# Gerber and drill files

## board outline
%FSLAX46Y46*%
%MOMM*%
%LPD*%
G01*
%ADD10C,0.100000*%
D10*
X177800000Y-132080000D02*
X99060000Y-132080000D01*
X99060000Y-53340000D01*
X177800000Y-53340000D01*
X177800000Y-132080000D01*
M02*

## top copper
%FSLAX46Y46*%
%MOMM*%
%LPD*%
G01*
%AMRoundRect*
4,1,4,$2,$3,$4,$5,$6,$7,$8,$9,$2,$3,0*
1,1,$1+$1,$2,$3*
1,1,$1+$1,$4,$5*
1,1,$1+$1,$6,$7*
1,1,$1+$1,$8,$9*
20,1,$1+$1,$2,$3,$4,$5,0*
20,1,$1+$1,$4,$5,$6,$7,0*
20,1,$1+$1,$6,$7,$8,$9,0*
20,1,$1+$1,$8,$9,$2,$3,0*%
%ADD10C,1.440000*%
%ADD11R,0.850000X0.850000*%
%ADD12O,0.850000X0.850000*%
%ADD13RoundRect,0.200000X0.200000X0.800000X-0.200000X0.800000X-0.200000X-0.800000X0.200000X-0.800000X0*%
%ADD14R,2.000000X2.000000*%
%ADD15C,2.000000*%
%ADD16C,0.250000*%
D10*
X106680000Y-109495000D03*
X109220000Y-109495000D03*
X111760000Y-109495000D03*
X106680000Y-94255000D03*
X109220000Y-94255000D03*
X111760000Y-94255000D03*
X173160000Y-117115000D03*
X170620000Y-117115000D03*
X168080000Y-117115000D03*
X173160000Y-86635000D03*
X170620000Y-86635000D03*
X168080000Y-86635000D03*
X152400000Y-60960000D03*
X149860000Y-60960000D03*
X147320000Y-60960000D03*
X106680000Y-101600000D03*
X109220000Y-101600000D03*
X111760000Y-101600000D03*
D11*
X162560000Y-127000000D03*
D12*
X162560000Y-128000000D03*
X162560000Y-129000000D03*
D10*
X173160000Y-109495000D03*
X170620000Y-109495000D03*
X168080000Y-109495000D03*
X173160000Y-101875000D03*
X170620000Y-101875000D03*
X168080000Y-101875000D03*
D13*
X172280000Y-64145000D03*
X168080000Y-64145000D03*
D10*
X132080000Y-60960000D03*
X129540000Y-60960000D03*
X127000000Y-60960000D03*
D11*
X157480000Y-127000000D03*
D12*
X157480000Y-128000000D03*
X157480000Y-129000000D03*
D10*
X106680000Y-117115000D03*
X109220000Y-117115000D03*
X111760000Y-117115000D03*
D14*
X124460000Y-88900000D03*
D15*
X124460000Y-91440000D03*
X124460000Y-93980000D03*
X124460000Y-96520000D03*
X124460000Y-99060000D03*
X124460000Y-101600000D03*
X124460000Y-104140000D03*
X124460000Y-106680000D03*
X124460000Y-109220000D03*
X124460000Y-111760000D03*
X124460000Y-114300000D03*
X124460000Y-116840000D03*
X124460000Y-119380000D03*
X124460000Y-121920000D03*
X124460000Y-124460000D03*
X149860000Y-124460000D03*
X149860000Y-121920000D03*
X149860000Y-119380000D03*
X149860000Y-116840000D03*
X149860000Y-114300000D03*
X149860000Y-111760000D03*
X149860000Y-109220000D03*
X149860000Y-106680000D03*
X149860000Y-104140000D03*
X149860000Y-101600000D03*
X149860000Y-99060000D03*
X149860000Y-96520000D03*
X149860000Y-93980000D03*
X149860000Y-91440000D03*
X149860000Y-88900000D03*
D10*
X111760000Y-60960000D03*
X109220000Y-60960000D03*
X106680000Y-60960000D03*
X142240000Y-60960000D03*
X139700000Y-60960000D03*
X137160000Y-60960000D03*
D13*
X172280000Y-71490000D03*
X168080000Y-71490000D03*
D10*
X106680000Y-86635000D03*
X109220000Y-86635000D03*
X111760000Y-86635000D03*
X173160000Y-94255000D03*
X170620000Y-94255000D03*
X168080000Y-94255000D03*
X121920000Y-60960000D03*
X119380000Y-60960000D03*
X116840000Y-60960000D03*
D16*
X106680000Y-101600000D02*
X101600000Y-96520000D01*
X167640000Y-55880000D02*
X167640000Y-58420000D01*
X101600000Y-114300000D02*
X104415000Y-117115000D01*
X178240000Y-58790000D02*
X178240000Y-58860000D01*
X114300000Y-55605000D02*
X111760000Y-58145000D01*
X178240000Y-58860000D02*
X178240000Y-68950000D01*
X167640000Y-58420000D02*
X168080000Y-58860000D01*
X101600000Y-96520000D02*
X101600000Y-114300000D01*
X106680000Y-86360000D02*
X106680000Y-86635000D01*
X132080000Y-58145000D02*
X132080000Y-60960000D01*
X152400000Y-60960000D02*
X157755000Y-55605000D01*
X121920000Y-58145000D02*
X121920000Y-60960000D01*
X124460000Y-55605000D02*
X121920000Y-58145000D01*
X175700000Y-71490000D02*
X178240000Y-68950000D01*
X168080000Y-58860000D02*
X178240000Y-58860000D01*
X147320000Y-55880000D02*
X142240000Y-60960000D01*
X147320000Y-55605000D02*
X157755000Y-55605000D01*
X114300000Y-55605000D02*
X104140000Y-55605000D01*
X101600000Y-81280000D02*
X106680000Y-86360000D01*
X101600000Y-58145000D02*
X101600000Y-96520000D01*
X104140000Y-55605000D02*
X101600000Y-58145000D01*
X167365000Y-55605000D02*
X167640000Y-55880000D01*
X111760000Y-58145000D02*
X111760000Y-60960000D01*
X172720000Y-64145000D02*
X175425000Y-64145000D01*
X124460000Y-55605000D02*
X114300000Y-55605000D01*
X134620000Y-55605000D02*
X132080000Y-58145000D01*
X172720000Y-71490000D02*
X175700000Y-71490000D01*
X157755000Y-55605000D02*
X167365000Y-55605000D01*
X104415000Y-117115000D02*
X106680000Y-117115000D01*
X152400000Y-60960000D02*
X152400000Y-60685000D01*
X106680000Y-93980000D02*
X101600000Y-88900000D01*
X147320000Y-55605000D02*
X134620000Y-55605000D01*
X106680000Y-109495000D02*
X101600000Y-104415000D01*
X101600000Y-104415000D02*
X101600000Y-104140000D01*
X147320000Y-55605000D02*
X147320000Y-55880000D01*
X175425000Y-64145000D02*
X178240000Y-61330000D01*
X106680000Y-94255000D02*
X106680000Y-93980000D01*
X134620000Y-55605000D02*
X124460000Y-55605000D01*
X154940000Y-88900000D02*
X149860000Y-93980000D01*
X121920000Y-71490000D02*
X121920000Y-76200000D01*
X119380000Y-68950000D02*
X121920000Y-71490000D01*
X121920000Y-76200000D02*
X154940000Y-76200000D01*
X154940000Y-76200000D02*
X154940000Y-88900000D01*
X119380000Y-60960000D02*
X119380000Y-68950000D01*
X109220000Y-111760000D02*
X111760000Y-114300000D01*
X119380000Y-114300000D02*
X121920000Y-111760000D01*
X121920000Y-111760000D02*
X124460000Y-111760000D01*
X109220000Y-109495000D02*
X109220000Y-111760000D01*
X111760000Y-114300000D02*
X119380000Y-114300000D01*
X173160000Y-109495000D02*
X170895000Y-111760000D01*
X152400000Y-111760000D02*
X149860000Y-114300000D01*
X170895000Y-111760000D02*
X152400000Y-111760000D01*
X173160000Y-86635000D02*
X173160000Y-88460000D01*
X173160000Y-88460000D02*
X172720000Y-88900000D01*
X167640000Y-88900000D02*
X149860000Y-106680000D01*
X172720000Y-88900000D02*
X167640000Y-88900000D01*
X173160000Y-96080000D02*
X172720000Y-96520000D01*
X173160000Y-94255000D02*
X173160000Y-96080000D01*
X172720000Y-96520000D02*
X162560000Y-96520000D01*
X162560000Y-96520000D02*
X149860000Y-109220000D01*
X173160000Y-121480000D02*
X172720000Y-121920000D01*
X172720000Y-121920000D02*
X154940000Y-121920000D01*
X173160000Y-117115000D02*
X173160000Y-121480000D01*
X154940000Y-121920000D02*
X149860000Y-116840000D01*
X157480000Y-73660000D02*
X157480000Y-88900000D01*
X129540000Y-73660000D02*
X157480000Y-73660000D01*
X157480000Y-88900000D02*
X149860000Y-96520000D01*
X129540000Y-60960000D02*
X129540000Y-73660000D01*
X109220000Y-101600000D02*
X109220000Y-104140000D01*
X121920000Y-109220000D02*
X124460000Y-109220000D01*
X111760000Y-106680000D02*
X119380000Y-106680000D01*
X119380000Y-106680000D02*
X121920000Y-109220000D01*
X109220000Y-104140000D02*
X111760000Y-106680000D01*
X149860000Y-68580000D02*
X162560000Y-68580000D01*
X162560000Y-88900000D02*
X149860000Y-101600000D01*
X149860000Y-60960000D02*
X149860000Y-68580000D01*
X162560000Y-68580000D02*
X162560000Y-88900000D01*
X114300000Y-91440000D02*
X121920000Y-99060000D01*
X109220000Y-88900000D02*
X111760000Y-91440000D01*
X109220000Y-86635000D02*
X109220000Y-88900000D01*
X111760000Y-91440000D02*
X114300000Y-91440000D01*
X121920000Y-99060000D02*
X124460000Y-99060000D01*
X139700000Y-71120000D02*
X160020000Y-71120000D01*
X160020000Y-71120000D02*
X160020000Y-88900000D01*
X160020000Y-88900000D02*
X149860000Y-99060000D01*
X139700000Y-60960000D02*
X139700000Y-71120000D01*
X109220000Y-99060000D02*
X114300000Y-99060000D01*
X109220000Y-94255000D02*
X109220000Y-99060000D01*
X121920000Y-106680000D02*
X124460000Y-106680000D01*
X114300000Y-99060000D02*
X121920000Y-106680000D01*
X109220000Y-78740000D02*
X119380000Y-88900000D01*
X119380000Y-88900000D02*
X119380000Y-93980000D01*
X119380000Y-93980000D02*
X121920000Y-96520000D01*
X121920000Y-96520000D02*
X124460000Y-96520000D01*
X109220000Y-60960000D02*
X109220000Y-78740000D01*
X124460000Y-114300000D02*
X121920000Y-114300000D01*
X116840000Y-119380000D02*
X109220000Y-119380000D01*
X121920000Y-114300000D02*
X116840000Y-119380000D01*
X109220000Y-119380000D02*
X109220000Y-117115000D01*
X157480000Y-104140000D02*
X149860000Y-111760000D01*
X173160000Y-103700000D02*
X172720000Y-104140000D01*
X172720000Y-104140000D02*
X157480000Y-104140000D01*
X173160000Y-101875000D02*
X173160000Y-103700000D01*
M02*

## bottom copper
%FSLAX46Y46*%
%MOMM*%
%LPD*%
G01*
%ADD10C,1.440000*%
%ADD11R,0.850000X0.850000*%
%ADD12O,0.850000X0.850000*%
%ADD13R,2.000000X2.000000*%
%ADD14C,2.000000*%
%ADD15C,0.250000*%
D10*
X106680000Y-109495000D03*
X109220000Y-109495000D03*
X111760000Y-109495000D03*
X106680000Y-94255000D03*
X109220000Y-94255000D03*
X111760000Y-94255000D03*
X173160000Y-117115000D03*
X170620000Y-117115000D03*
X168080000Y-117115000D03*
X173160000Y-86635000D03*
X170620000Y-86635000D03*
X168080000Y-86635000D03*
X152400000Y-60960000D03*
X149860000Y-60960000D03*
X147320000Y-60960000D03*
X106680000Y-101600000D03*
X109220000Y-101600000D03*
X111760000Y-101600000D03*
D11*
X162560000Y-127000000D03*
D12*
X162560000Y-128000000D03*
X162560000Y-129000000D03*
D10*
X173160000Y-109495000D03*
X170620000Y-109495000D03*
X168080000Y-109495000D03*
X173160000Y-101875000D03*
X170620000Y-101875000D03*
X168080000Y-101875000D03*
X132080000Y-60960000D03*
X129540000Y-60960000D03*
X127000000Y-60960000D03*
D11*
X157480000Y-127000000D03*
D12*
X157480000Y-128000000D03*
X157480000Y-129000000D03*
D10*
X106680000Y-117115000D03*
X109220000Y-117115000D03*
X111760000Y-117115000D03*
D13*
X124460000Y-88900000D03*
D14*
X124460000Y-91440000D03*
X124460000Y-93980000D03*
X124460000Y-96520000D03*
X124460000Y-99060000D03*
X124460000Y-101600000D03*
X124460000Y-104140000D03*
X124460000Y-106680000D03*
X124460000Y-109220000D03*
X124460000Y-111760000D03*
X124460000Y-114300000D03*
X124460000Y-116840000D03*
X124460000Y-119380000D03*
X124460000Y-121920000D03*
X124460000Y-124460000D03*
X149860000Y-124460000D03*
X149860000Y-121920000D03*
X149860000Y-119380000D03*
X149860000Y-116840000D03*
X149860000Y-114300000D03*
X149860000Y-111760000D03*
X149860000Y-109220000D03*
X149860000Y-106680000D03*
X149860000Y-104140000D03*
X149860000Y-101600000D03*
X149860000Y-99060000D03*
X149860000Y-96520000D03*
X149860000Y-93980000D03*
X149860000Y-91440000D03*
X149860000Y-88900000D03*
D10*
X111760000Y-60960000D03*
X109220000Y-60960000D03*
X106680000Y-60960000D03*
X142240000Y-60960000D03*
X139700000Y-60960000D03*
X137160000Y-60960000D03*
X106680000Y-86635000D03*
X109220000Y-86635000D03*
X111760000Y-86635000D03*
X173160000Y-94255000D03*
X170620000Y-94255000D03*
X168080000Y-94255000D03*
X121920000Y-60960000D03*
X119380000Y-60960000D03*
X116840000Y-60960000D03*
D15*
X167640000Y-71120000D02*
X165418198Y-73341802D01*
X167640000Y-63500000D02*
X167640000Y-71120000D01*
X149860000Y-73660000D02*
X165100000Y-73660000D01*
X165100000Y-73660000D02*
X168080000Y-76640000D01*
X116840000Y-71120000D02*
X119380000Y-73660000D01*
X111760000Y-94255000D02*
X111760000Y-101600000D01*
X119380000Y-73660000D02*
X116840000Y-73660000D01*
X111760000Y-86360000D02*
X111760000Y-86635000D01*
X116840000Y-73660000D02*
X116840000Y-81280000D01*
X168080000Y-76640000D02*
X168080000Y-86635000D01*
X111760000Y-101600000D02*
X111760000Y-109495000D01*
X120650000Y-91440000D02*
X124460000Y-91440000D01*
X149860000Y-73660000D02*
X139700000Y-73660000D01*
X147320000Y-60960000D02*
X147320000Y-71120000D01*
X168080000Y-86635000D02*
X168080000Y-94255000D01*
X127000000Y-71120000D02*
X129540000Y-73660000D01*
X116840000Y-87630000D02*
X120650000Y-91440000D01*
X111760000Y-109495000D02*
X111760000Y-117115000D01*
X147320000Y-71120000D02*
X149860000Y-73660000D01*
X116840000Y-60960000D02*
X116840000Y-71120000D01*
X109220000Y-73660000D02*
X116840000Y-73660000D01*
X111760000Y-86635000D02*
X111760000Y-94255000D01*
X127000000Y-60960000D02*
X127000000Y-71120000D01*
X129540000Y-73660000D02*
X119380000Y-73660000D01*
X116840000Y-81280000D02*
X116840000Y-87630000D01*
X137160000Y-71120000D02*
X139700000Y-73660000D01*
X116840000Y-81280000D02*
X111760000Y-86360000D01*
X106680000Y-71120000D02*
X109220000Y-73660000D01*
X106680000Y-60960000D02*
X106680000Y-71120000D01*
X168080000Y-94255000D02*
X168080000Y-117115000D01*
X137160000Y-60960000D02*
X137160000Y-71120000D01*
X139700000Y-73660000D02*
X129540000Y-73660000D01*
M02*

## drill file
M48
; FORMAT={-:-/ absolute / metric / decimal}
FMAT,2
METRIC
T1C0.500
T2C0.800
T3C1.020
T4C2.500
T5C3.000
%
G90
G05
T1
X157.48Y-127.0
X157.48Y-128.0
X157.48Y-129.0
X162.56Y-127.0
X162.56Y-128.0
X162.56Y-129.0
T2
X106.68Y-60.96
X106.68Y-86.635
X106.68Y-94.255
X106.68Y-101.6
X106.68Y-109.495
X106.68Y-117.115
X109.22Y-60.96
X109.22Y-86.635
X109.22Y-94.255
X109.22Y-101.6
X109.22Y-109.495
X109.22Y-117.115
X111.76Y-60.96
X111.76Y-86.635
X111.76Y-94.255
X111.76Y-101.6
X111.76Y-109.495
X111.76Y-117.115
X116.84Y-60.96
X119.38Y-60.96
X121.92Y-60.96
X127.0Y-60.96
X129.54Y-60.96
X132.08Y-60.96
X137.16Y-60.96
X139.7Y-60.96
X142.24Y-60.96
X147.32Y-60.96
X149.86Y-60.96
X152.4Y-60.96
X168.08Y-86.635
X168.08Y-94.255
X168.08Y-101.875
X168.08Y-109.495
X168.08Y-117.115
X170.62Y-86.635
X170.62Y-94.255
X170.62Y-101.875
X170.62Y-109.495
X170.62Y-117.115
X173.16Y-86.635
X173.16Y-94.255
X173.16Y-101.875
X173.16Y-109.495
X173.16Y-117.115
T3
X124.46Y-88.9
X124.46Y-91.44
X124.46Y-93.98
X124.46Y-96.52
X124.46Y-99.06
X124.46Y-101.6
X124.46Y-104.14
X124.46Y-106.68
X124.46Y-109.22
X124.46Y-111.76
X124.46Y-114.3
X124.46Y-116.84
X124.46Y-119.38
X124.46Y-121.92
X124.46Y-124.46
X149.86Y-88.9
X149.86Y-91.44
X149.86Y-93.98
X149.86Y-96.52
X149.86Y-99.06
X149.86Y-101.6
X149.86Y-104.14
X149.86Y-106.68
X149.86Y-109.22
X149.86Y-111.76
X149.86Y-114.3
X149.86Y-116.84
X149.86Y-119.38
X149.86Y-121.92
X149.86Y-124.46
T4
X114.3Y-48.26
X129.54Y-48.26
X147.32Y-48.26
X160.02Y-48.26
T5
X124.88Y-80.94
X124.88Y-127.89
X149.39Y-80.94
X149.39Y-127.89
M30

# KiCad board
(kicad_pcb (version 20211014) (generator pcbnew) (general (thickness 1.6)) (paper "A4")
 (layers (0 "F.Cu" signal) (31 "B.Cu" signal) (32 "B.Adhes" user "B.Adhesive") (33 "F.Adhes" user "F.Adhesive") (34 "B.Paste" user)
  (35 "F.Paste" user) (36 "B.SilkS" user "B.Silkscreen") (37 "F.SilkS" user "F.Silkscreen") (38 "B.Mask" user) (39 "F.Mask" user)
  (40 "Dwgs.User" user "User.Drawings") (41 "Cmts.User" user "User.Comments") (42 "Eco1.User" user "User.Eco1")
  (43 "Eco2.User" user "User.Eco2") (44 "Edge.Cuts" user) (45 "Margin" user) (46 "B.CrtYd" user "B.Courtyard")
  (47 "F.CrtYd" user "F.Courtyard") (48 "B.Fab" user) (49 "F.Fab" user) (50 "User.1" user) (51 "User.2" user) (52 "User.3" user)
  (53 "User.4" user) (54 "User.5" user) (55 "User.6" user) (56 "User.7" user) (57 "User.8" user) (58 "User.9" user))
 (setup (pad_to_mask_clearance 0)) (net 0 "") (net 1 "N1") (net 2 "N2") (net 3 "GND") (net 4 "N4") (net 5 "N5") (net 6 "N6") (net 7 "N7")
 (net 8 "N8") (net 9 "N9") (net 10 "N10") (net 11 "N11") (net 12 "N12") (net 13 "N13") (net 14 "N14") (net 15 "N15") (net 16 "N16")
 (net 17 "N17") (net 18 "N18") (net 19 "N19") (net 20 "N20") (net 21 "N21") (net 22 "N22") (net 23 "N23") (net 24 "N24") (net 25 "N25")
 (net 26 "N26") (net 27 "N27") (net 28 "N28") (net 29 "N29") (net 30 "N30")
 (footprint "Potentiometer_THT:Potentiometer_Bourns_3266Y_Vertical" (layer "F.Cu") (at 106.68 109.495 180)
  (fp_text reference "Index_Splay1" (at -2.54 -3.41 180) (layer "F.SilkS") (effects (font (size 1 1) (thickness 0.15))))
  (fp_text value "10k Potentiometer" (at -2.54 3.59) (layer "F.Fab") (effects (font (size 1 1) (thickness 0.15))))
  (pad "1" thru_hole circle (at 0 0 180) (size 1.44 1.44) (drill 0.8) (layers *.Cu *.Mask) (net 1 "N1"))
  (pad "2" thru_hole circle (at -2.54 0 180) (size 1.44 1.44) (drill 0.8) (layers *.Cu *.Mask) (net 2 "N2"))
  (pad "3" thru_hole circle (at -5.08 0 180) (size 1.44 1.44) (drill 0.8) (layers *.Cu *.Mask) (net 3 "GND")))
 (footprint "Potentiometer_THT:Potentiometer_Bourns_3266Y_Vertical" (layer "F.Cu") (at 106.68 94.255 180)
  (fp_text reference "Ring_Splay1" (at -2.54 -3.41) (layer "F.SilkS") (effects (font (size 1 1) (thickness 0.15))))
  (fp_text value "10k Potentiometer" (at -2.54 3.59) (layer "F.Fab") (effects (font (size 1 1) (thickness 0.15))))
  (pad "1" thru_hole circle (at 0 0 180) (size 1.44 1.44) (drill 0.8) (layers *.Cu *.Mask) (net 1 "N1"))
  (pad "2" thru_hole circle (at -2.54 0 180) (size 1.44 1.44) (drill 0.8) (layers *.Cu *.Mask) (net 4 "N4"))
  (pad "3" thru_hole circle (at -5.08 0 180) (size 1.44 1.44) (drill 0.8) (layers *.Cu *.Mask) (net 3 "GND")))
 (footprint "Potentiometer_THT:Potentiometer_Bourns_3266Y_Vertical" (layer "F.Cu") (at 173.16 117.115)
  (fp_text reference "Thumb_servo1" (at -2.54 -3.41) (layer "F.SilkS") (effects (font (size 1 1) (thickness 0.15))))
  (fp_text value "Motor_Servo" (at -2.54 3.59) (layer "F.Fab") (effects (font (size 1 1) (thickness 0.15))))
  (pad "1" thru_hole circle (at 0 0) (size 1.44 1.44) (drill 0.8) (layers *.Cu *.Mask) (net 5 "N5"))
  (pad "2" thru_hole circle (at -2.54 0) (size 1.44 1.44) (drill 0.8) (layers *.Cu *.Mask) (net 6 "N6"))
  (pad "3" thru_hole circle (at -5.08 0) (size 1.44 1.44) (drill 0.8) (layers *.Cu *.Mask) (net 3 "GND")))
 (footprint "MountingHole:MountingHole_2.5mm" (layer "F.Cu") (at 160.02 48.26)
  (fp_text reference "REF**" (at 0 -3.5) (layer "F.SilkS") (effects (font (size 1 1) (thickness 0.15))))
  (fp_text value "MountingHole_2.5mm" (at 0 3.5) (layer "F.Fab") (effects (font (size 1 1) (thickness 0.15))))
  (pad "" np_thru_hole circle (at 0 0) (size 2.5 2.5) (drill 2.5) (layers *.Cu *.Mask)))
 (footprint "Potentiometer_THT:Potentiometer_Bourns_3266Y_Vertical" (layer "F.Cu") (at 173.16 86.635)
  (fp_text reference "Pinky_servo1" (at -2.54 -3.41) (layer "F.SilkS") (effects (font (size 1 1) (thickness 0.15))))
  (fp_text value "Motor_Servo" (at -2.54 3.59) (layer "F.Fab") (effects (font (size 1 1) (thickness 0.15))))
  (pad "1" thru_hole circle (at 0 0) (size 1.44 1.44) (drill 0.8) (layers *.Cu *.Mask) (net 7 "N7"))
  (pad "2" thru_hole circle (at -2.54 0) (size 1.44 1.44) (drill 0.8) (layers *.Cu *.Mask) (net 6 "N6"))
  (pad "3" thru_hole circle (at -5.08 0) (size 1.44 1.44) (drill 0.8) (layers *.Cu *.Mask) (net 3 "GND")))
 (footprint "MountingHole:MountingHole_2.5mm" (layer "F.Cu") (at 114.3 48.26)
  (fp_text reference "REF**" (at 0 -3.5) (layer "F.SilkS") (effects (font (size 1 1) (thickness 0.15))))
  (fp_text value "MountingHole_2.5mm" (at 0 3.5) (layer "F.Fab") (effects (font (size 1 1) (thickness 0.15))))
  (pad "" np_thru_hole circle (at 0 0) (size 2.5 2.5) (drill 2.5) (layers *.Cu *.Mask)))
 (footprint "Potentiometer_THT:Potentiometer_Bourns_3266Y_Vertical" (layer "F.Cu") (at 152.4 60.96)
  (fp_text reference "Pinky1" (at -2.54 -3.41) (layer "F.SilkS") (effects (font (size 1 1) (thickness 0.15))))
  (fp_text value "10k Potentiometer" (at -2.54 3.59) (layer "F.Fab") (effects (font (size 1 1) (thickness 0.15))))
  (pad "1" thru_hole circle (at 0 0) (size 1.44 1.44) (drill 0.8) (layers *.Cu *.Mask) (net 1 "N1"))
  (pad "2" thru_hole circle (at -2.54 0) (size 1.44 1.44) (drill 0.8) (layers *.Cu *.Mask) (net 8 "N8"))
  (pad "3" thru_hole circle (at -5.08 0) (size 1.44 1.44) (drill 0.8) (layers *.Cu *.Mask) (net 3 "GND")))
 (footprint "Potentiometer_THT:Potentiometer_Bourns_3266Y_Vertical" (layer "F.Cu") (at 106.68 101.6 180)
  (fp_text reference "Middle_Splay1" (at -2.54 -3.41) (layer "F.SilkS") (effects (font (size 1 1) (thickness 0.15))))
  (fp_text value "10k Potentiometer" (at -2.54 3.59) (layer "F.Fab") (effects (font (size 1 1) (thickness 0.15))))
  (pad "1" thru_hole circle (at 0 0 180) (size 1.44 1.44) (drill 0.8) (layers *.Cu *.Mask) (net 1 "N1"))
  (pad "2" thru_hole circle (at -2.54 0 180) (size 1.44 1.44) (drill 0.8) (layers *.Cu *.Mask) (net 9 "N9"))
  (pad "3" thru_hole circle (at -5.08 0 180) (size 1.44 1.44) (drill 0.8) (layers *.Cu *.Mask) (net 3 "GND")))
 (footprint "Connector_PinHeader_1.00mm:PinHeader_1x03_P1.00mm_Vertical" (layer "F.Cu") (at 162.56 127)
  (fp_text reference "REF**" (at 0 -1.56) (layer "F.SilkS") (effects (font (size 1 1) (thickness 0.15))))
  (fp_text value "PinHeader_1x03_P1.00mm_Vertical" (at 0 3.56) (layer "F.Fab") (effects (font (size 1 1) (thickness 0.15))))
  (pad "1" thru_hole rect (at 0 0) (size 0.85 0.85) (drill 0.5) (layers *.Cu *.Mask))
  (pad "2" thru_hole oval (at 0 1) (size 0.85 0.85) (drill 0.5) (layers *.Cu *.Mask))
  (pad "3" thru_hole oval (at 0 2) (size 0.85 0.85) (drill 0.5) (layers *.Cu *.Mask)))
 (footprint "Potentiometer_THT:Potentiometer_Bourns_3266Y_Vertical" (layer "F.Cu") (at 173.16 109.495)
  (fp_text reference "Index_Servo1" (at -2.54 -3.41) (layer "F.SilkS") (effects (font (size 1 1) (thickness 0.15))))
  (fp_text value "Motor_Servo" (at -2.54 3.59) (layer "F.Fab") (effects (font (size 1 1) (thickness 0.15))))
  (pad "1" thru_hole circle (at 0 0) (size 1.44 1.44) (drill 0.8) (layers *.Cu *.Mask) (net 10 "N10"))
  (pad "2" thru_hole circle (at -2.54 0) (size 1.44 1.44) (drill 0.8) (layers *.Cu *.Mask) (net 6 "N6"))
  (pad "3" thru_hole circle (at -5.08 0) (size 1.44 1.44) (drill 0.8) (layers *.Cu *.Mask) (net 3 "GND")))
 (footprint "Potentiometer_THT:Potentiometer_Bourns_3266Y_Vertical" (layer "F.Cu") (at 173.16 101.875)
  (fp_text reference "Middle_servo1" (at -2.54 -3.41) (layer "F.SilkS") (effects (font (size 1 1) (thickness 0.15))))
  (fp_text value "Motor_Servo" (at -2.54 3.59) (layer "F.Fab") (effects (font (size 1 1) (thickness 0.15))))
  (pad "1" thru_hole circle (at 0 0) (size 1.44 1.44) (drill 0.8) (layers *.Cu *.Mask) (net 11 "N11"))
  (pad "2" thru_hole circle (at -2.54 0) (size 1.44 1.44) (drill 0.8) (layers *.Cu *.Mask) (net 6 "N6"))
  (pad "3" thru_hole circle (at -5.08 0) (size 1.44 1.44) (drill 0.8) (layers *.Cu *.Mask) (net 3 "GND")))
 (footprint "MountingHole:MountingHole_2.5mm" (layer "F.Cu") (at 147.32 48.26)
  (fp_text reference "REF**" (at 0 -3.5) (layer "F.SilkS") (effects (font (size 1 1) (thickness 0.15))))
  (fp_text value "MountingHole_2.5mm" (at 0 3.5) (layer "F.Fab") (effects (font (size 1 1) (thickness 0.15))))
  (pad "" np_thru_hole circle (at 0 0) (size 2.5 2.5) (drill 2.5) (layers *.Cu *.Mask)))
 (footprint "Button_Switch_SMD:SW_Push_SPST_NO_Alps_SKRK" (layer "F.Cu") (at 170.18 64.145 180)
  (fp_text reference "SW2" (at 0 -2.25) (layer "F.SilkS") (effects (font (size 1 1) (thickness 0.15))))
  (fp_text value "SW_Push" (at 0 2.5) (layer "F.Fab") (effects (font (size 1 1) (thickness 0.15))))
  (pad "1" smd roundrect (at -2.1 0 180) (size 0.8 2) (layers "F.Cu" "F.Paste" "F.Mask") (roundrect_rratio 0.25) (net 1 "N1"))
  (pad "2" smd roundrect (at 2.1 0 180) (size 0.8 2) (layers "F.Cu" "F.Paste" "F.Mask") (roundrect_rratio 0.25) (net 3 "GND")))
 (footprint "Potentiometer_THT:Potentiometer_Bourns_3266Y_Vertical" (layer "F.Cu") (at 132.08 60.96)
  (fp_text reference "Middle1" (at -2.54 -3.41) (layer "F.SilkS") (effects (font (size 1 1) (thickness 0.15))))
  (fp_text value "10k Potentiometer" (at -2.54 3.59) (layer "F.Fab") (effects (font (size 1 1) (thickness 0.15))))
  (pad "1" thru_hole circle (at 0 0) (size 1.44 1.44) (drill 0.8) (layers *.Cu *.Mask) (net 1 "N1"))
  (pad "2" thru_hole circle (at -2.54 0) (size 1.44 1.44) (drill 0.8) (layers *.Cu *.Mask) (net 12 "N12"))
  (pad "3" thru_hole circle (at -5.08 0) (size 1.44 1.44) (drill 0.8) (layers *.Cu *.Mask) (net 3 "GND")))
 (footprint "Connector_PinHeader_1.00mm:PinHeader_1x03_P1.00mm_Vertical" (layer "F.Cu") (at 157.48 127)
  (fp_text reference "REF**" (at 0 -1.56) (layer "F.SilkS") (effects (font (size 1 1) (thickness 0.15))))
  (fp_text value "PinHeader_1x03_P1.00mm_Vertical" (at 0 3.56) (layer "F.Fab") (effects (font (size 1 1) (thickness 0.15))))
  (pad "1" thru_hole rect (at 0 0) (size 0.85 0.85) (drill 0.5) (layers *.Cu *.Mask))
  (pad "2" thru_hole oval (at 0 1) (size 0.85 0.85) (drill 0.5) (layers *.Cu *.Mask))
  (pad "3" thru_hole oval (at 0 2) (size 0.85 0.85) (drill 0.5) (layers *.Cu *.Mask)))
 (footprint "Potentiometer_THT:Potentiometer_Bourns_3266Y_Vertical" (layer "F.Cu") (at 106.68 117.115 180)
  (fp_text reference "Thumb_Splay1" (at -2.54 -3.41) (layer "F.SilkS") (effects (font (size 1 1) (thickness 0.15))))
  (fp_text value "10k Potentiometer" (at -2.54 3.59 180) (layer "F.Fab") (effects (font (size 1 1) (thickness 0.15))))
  (pad "1" thru_hole circle (at 0 0 180) (size 1.44 1.44) (drill 0.8) (layers *.Cu *.Mask) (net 1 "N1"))
  (pad "2" thru_hole circle (at -2.54 0 180) (size 1.44 1.44) (drill 0.8) (layers *.Cu *.Mask) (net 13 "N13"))
  (pad "3" thru_hole circle (at -5.08 0 180) (size 1.44 1.44) (drill 0.8) (layers *.Cu *.Mask) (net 3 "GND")))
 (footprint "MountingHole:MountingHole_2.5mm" (layer "F.Cu") (at 129.54 48.26)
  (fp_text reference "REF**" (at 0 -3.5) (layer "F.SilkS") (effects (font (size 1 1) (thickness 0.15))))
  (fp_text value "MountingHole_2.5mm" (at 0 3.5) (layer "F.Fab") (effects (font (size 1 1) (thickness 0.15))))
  (pad "" np_thru_hole circle (at 0 0) (size 2.5 2.5) (drill 2.5) (layers *.Cu *.Mask)))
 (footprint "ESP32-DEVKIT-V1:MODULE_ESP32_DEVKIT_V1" (layer "F.Cu") (at 137.16 104.415)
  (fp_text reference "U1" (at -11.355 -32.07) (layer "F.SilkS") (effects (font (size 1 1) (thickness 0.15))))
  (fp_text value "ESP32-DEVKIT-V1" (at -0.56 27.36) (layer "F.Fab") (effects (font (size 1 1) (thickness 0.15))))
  (pad "" np_thru_hole circle (at -12.28 -23.475) (size 3 3) (drill 3) (layers *.Cu *.Mask))
  (pad "" np_thru_hole circle (at 12.23 23.475) (size 3 3) (drill 3) (layers *.Cu *.Mask))
  (pad "" np_thru_hole circle (at 12.23 -23.475) (size 3 3) (drill 3) (layers *.Cu *.Mask))
  (pad "" np_thru_hole circle (at -12.28 23.475) (size 3 3) (drill 3) (layers *.Cu *.Mask))
  (pad "1" thru_hole rect (at -12.7 -15.515) (size 2 2) (drill 1.02) (layers *.Cu *.Mask) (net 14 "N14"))
  (pad "2" thru_hole circle (at -12.7 -12.975) (size 2 2) (drill 1.02) (layers *.Cu *.Mask) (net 3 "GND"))
  (pad "3" thru_hole circle (at -12.7 -10.435) (size 2 2) (drill 1.02) (layers *.Cu *.Mask) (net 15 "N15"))
  (pad "4" thru_hole circle (at -12.7 -7.895) (size 2 2) (drill 1.02) (layers *.Cu *.Mask) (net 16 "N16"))
  (pad "5" thru_hole circle (at -12.7 -5.355) (size 2 2) (drill 1.02) (layers *.Cu *.Mask) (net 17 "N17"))
  (pad "6" thru_hole circle (at -12.7 -2.815) (size 2 2) (drill 1.02) (layers *.Cu *.Mask) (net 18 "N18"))
  (pad "7" thru_hole circle (at -12.7 -0.275) (size 2 2) (drill 1.02) (layers *.Cu *.Mask) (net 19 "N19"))
  (pad "8" thru_hole circle (at -12.7 2.265) (size 2 2) (drill 1.02) (layers *.Cu *.Mask) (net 4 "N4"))
  (pad "9" thru_hole circle (at -12.7 4.805) (size 2 2) (drill 1.02) (layers *.Cu *.Mask) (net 9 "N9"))
  (pad "10" thru_hole circle (at -12.7 7.345) (size 2 2) (drill 1.02) (layers *.Cu *.Mask) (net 2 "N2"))
  (pad "11" thru_hole circle (at -12.7 9.885) (size 2 2) (drill 1.02) (layers *.Cu *.Mask) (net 13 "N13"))
  (pad "12" thru_hole circle (at -12.7 12.425) (size 2 2) (drill 1.02) (layers *.Cu *.Mask) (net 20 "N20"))
  (pad "13" thru_hole circle (at -12.7 14.965) (size 2 2) (drill 1.02) (layers *.Cu *.Mask) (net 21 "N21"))
  (pad "14" thru_hole circle (at -12.7 17.505) (size 2 2) (drill 1.02) (layers *.Cu *.Mask) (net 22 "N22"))
  (pad "15" thru_hole circle (at -12.7 20.045) (size 2 2) (drill 1.02) (layers *.Cu *.Mask) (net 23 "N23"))
  (pad "16" thru_hole circle (at 12.7 20.045) (size 2 2) (drill 1.02) (layers *.Cu *.Mask) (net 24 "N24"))
  (pad "17" thru_hole circle (at 12.7 17.505) (size 2 2) (drill 1.02) (layers *.Cu *.Mask) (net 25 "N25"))
  (pad "18" thru_hole circle (at 12.7 14.965) (size 2 2) (drill 1.02) (layers *.Cu *.Mask) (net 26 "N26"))
  (pad "19" thru_hole circle (at 12.7 12.425) (size 2 2) (drill 1.02) (layers *.Cu *.Mask) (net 5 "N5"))
  (pad "20" thru_hole circle (at 12.7 9.885) (size 2 2) (drill 1.02) (layers *.Cu *.Mask) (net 10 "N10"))
  (pad "21" thru_hole circle (at 12.7 7.345) (size 2 2) (drill 1.02) (layers *.Cu *.Mask) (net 11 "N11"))
  (pad "22" thru_hole circle (at 12.7 4.805) (size 2 2) (drill 1.02) (layers *.Cu *.Mask) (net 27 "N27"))
  (pad "23" thru_hole circle (at 12.7 2.265) (size 2 2) (drill 1.02) (layers *.Cu *.Mask) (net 7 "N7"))
  (pad "24" thru_hole circle (at 12.7 -0.275) (size 2 2) (drill 1.02) (layers *.Cu *.Mask) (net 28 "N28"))
  (pad "25" thru_hole circle (at 12.7 -2.815) (size 2 2) (drill 1.02) (layers *.Cu *.Mask) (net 8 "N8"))
  (pad "26" thru_hole circle (at 12.7 -5.355) (size 2 2) (drill 1.02) (layers *.Cu *.Mask) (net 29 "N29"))
  (pad "27" thru_hole circle (at 12.7 -7.895) (size 2 2) (drill 1.02) (layers *.Cu *.Mask) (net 12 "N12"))
  (pad "28" thru_hole circle (at 12.7 -10.435) (size 2 2) (drill 1.02) (layers *.Cu *.Mask) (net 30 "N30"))
  (pad "29" thru_hole circle (at 12.7 -12.975) (size 2 2) (drill 1.02) (layers *.Cu *.Mask) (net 3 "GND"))
  (pad "30" thru_hole circle (at 12.7 -15.515) (size 2 2) (drill 1.02) (layers *.Cu *.Mask) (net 1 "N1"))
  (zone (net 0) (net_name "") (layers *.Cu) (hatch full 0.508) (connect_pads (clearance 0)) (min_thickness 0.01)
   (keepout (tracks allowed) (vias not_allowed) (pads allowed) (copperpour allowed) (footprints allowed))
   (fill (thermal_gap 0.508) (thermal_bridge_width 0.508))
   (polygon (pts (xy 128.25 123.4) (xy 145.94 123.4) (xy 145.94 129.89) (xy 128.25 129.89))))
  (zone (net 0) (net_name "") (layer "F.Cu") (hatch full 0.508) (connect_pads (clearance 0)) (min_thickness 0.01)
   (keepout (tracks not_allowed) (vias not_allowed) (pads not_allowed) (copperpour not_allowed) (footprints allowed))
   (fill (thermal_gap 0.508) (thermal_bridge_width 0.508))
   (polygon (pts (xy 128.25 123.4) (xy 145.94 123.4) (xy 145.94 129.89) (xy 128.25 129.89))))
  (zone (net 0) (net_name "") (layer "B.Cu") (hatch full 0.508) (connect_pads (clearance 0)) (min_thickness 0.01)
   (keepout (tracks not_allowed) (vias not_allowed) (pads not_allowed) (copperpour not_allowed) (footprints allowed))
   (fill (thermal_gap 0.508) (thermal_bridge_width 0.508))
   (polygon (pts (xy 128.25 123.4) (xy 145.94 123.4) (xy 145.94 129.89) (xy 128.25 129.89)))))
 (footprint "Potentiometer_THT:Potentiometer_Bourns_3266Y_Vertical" (layer "F.Cu") (at 111.76 60.96)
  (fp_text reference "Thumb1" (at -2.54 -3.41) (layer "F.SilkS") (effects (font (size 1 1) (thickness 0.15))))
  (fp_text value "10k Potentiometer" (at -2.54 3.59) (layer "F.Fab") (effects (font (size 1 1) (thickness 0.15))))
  (pad "1" thru_hole circle (at 0 0) (size 1.44 1.44) (drill 0.8) (layers *.Cu *.Mask) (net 1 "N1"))
  (pad "2" thru_hole circle (at -2.54 0) (size 1.44 1.44) (drill 0.8) (layers *.Cu *.Mask) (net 16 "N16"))
  (pad "3" thru_hole circle (at -5.08 0) (size 1.44 1.44) (drill 0.8) (layers *.Cu *.Mask) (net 3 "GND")))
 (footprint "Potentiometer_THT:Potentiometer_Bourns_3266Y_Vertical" (layer "F.Cu") (at 142.24 60.96)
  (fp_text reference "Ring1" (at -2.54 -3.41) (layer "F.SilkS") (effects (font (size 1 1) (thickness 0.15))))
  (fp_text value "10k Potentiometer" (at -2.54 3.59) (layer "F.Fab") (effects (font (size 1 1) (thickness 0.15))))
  (pad "1" thru_hole circle (at 0 0) (size 1.44 1.44) (drill 0.8) (layers *.Cu *.Mask) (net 1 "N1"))
  (pad "2" thru_hole circle (at -2.54 0) (size 1.44 1.44) (drill 0.8) (layers *.Cu *.Mask) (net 29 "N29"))
  (pad "3" thru_hole circle (at -5.08 0) (size 1.44 1.44) (drill 0.8) (layers *.Cu *.Mask) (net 3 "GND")))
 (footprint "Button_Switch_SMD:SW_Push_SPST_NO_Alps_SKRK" (layer "F.Cu") (at 170.18 71.49 180)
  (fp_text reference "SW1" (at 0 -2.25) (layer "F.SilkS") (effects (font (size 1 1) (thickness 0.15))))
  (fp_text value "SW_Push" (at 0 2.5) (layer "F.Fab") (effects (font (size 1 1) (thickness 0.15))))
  (pad "1" smd roundrect (at -2.1 0 180) (size 0.8 2) (layers "F.Cu" "F.Paste" "F.Mask") (roundrect_rratio 0.25) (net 1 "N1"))
  (pad "2" smd roundrect (at 2.1 0 180) (size 0.8 2) (layers "F.Cu" "F.Paste" "F.Mask") (roundrect_rratio 0.25) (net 3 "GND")))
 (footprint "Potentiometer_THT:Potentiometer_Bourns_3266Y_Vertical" (layer "F.Cu") (at 106.68 86.635 180)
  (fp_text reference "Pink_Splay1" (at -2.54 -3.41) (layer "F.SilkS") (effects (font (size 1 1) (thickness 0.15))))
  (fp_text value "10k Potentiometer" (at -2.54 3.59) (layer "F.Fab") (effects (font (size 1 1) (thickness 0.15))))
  (pad "1" thru_hole circle (at 0 0 180) (size 1.44 1.44) (drill 0.8) (layers *.Cu *.Mask) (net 1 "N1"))
  (pad "2" thru_hole circle (at -2.54 0 180) (size 1.44 1.44) (drill 0.8) (layers *.Cu *.Mask) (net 17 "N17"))
  (pad "3" thru_hole circle (at -5.08 0 180) (size 1.44 1.44) (drill 0.8) (layers *.Cu *.Mask) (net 3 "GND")))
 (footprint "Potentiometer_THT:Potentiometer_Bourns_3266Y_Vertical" (layer "F.Cu") (at 173.16 94.255)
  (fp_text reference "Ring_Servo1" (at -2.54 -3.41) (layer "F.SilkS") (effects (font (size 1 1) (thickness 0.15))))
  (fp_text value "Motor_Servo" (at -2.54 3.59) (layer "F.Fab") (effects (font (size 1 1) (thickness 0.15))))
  (pad "1" thru_hole circle (at 0 0) (size 1.44 1.44) (drill 0.8) (layers *.Cu *.Mask) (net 27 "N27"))
  (pad "2" thru_hole circle (at -2.54 0) (size 1.44 1.44) (drill 0.8) (layers *.Cu *.Mask) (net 6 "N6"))
  (pad "3" thru_hole circle (at -5.08 0) (size 1.44 1.44) (drill 0.8) (layers *.Cu *.Mask) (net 3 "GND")))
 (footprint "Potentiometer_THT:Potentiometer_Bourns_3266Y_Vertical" (layer "F.Cu") (at 121.92 60.96)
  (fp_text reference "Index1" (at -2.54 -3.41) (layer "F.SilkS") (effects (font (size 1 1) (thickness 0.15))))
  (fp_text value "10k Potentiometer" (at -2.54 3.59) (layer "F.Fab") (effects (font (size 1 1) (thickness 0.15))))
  (pad "1" thru_hole circle (at 0 0) (size 1.44 1.44) (drill 0.8) (layers *.Cu *.Mask) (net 1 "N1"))
  (pad "2" thru_hole circle (at -2.54 0) (size 1.44 1.44) (drill 0.8) (layers *.Cu *.Mask) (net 30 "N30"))
  (pad "3" thru_hole circle (at -5.08 0) (size 1.44 1.44) (drill 0.8) (layers *.Cu *.Mask) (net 3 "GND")))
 (gr_poly (pts (xy 177.8 132.08) (xy 99.06 132.08) (xy 99.06 53.34) (xy 177.8 53.34)) (layer "Edge.Cuts") (width 0.1) (fill none))
 (segment (start 167.64 71.12) (end 165.418198 73.341802) (width 0.25) (layer "B.Cu") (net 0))
 (segment (start 167.64 63.5) (end 167.64 71.12) (width 0.25) (layer "B.Cu") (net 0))
 (segment (start 106.68 101.6) (end 101.6 96.52) (width 0.25) (layer "F.Cu") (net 1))
 (segment (start 167.64 55.88) (end 167.64 58.42) (width 0.25) (layer "F.Cu") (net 1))
 (segment (start 101.6 114.3) (end 104.415 117.115) (width 0.25) (layer "F.Cu") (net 1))
 (segment (start 178.24 58.79) (end 178.24 58.86) (width 0.25) (layer "F.Cu") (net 1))
 (segment (start 114.3 55.605) (end 111.76 58.145) (width 0.25) (layer "F.Cu") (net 1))
 (segment (start 178.24 58.86) (end 178.24 68.95) (width 0.25) (layer "F.Cu") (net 1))
 (segment (start 167.64 58.42) (end 168.08 58.86) (width 0.25) (layer "F.Cu") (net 1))
 (segment (start 101.6 96.52) (end 101.6 114.3) (width 0.25) (layer "F.Cu") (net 1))
 (segment (start 106.68 86.36) (end 106.68 86.635) (width 0.25) (layer "F.Cu") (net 1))
 (segment (start 132.08 58.145) (end 132.08 60.96) (width 0.25) (layer "F.Cu") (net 1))
 (segment (start 152.4 60.96) (end 157.755 55.605) (width 0.25) (layer "F.Cu") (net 1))
 (segment (start 121.92 58.145) (end 121.92 60.96) (width 0.25) (layer "F.Cu") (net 1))
 (segment (start 124.46 55.605) (end 121.92 58.145) (width 0.25) (layer "F.Cu") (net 1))
 (segment (start 175.7 71.49) (end 178.24 68.95) (width 0.25) (layer "F.Cu") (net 1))
 (segment (start 168.08 58.86) (end 178.24 58.86) (width 0.25) (layer "F.Cu") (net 1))
 (segment (start 147.32 55.88) (end 142.24 60.96) (width 0.25) (layer "F.Cu") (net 1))
 (segment (start 147.32 55.605) (end 157.755 55.605) (width 0.25) (layer "F.Cu") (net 1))
 (segment (start 114.3 55.605) (end 104.14 55.605) (width 0.25) (layer "F.Cu") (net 1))
 (segment (start 101.6 81.28) (end 106.68 86.36) (width 0.25) (layer "F.Cu") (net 1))
 (segment (start 101.6 58.145) (end 101.6 96.52) (width 0.25) (layer "F.Cu") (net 1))
 (segment (start 104.14 55.605) (end 101.6 58.145) (width 0.25) (layer "F.Cu") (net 1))
 (segment (start 167.365 55.605) (end 167.64 55.88) (width 0.25) (layer "F.Cu") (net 1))
 (segment (start 111.76 58.145) (end 111.76 60.96) (width 0.25) (layer "F.Cu") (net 1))
 (segment (start 172.72 64.145) (end 175.425 64.145) (width 0.25) (layer "F.Cu") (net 1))
 (segment (start 124.46 55.605) (end 114.3 55.605) (width 0.25) (layer "F.Cu") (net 1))
 (segment (start 134.62 55.605) (end 132.08 58.145) (width 0.25) (layer "F.Cu") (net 1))
 (segment (start 172.72 71.49) (end 175.7 71.49) (width 0.25) (layer "F.Cu") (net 1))
 (segment (start 157.755 55.605) (end 167.365 55.605) (width 0.25) (layer "F.Cu") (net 1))
 (segment (start 104.415 117.115) (end 106.68 117.115) (width 0.25) (layer "F.Cu") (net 1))
 (segment (start 152.4 60.96) (end 152.4 60.685) (width 0.25) (layer "F.Cu") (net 1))
 (segment (start 106.68 93.98) (end 101.6 88.9) (width 0.25) (layer "F.Cu") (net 1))
 (segment (start 147.32 55.605) (end 134.62 55.605) (width 0.25) (layer "F.Cu") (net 1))
 (segment (start 106.68 109.495) (end 101.6 104.415) (width 0.25) (layer "F.Cu") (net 1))
 (segment (start 101.6 104.415) (end 101.6 104.14) (width 0.25) (layer "F.Cu") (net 1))
 (segment (start 147.32 55.605) (end 147.32 55.88) (width 0.25) (layer "F.Cu") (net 1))
 (segment (start 175.425 64.145) (end 178.24 61.33) (width 0.25) (layer "F.Cu") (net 1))
 (segment (start 106.68 94.255) (end 106.68 93.98) (width 0.25) (layer "F.Cu") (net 1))
 (segment (start 134.62 55.605) (end 124.46 55.605) (width 0.25) (layer "F.Cu") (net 1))
 (segment (start 154.94 88.9) (end 149.86 93.98) (width 0.25) (layer "F.Cu") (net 30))
 (segment (start 121.92 71.49) (end 121.92 76.2) (width 0.25) (layer "F.Cu") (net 30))
 (segment (start 119.38 68.95) (end 121.92 71.49) (width 0.25) (layer "F.Cu") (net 30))
 (segment (start 121.92 76.2) (end 154.94 76.2) (width 0.25) (layer "F.Cu") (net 30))
 (segment (start 154.94 76.2) (end 154.94 88.9) (width 0.25) (layer "F.Cu") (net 30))
 (segment (start 119.38 60.96) (end 119.38 68.95) (width 0.25) (layer "F.Cu") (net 30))
 (segment (start 149.86 73.66) (end 165.1 73.66) (width 0.25) (layer "B.Cu") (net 3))
 (segment (start 165.1 73.66) (end 168.08 76.64) (width 0.25) (layer "B.Cu") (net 3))
 (segment (start 116.84 71.12) (end 119.38 73.66) (width 0.25) (layer "B.Cu") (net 3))
 (segment (start 111.76 94.255) (end 111.76 101.6) (width 0.25) (layer "B.Cu") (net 3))
 (segment (start 119.38 73.66) (end 116.84 73.66) (width 0.25) (layer "B.Cu") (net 3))
 (segment (start 111.76 86.36) (end 111.76 86.635) (width 0.25) (layer "B.Cu") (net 3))
 (segment (start 116.84 73.66) (end 116.84 81.28) (width 0.25) (layer "B.Cu") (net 3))
 (segment (start 168.08 76.64) (end 168.08 86.635) (width 0.25) (layer "B.Cu") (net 3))
 (segment (start 111.76 101.6) (end 111.76 109.495) (width 0.25) (layer "B.Cu") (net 3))
 (segment (start 120.65 91.44) (end 124.46 91.44) (width 0.25) (layer "B.Cu") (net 3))
 (segment (start 149.86 73.66) (end 139.7 73.66) (width 0.25) (layer "B.Cu") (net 3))
 (segment (start 147.32 60.96) (end 147.32 71.12) (width 0.25) (layer "B.Cu") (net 3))
 (segment (start 168.08 86.635) (end 168.08 94.255) (width 0.25) (layer "B.Cu") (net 3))
 (segment (start 127 71.12) (end 129.54 73.66) (width 0.25) (layer "B.Cu") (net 3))
 (segment (start 116.84 87.63) (end 120.65 91.44) (width 0.25) (layer "B.Cu") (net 3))
 (segment (start 111.76 109.495) (end 111.76 117.115) (width 0.25) (layer "B.Cu") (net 3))
 (segment (start 147.32 71.12) (end 149.86 73.66) (width 0.25) (layer "B.Cu") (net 3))
 (segment (start 116.84 60.96) (end 116.84 71.12) (width 0.25) (layer "B.Cu") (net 3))
 (segment (start 109.22 73.66) (end 116.84 73.66) (width 0.25) (layer "B.Cu") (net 3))
 (segment (start 111.76 86.635) (end 111.76 94.255) (width 0.25) (layer "B.Cu") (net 3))
 (segment (start 127 60.96) (end 127 71.12) (width 0.25) (layer "B.Cu") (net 3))
 (segment (start 129.54 73.66) (end 119.38 73.66) (width 0.25) (layer "B.Cu") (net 3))
 (segment (start 116.84 81.28) (end 116.84 87.63) (width 0.25) (layer "B.Cu") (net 3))
 (segment (start 137.16 71.12) (end 139.7 73.66) (width 0.25) (layer "B.Cu") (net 3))
 (segment (start 116.84 81.28) (end 111.76 86.36) (width 0.25) (layer "B.Cu") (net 3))
 (segment (start 106.68 71.12) (end 109.22 73.66) (width 0.25) (layer "B.Cu") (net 3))
 (segment (start 106.68 60.96) (end 106.68 71.12) (width 0.25) (layer "B.Cu") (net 3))
 (segment (start 168.08 94.255) (end 168.08 117.115) (width 0.25) (layer "B.Cu") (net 3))
 (segment (start 137.16 60.96) (end 137.16 71.12) (width 0.25) (layer "B.Cu") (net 3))
 (segment (start 139.7 73.66) (end 129.54 73.66) (width 0.25) (layer "B.Cu") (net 3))
 (segment (start 109.22 111.76) (end 111.76 114.3) (width 0.25) (layer "F.Cu") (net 2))
 (segment (start 119.38 114.3) (end 121.92 111.76) (width 0.25) (layer "F.Cu") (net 2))
 (segment (start 121.92 111.76) (end 124.46 111.76) (width 0.25) (layer "F.Cu") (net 2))
 (segment (start 109.22 109.495) (end 109.22 111.76) (width 0.25) (layer "F.Cu") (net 2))
 (segment (start 111.76 114.3) (end 119.38 114.3) (width 0.25) (layer "F.Cu") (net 2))
 (segment (start 173.16 109.495) (end 170.895 111.76) (width 0.25) (layer "F.Cu") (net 10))
 (segment (start 152.4 111.76) (end 149.86 114.3) (width 0.25) (layer "F.Cu") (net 10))
 (segment (start 170.895 111.76) (end 152.4 111.76) (width 0.25) (layer "F.Cu") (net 10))
 (segment (start 173.16 86.635) (end 173.16 88.46) (width 0.25) (layer "F.Cu") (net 7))
 (segment (start 173.16 88.46) (end 172.72 88.9) (width 0.25) (layer "F.Cu") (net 7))
 (segment (start 167.64 88.9) (end 149.86 106.68) (width 0.25) (layer "F.Cu") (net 7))
 (segment (start 172.72 88.9) (end 167.64 88.9) (width 0.25) (layer "F.Cu") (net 7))
 (segment (start 173.16 96.08) (end 172.72 96.52) (width 0.25) (layer "F.Cu") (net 27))
 (segment (start 173.16 94.255) (end 173.16 96.08) (width 0.25) (layer "F.Cu") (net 27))
 (segment (start 172.72 96.52) (end 162.56 96.52) (width 0.25) (layer "F.Cu") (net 27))
 (segment (start 162.56 96.52) (end 149.86 109.22) (width 0.25) (layer "F.Cu") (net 27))
 (segment (start 173.16 121.48) (end 172.72 121.92) (width 0.25) (layer "F.Cu") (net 5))
 (segment (start 172.72 121.92) (end 154.94 121.92) (width 0.25) (layer "F.Cu") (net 5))
 (segment (start 173.16 117.115) (end 173.16 121.48) (width 0.25) (layer "F.Cu") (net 5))
 (segment (start 154.94 121.92) (end 149.86 116.84) (width 0.25) (layer "F.Cu") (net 5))
 (segment (start 157.48 73.66) (end 157.48 88.9) (width 0.25) (layer "F.Cu") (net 12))
 (segment (start 129.54 73.66) (end 157.48 73.66) (width 0.25) (layer "F.Cu") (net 12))
 (segment (start 157.48 88.9) (end 149.86 96.52) (width 0.25) (layer "F.Cu") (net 12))
 (segment (start 129.54 60.96) (end 129.54 73.66) (width 0.25) (layer "F.Cu") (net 12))
 (segment (start 109.22 101.6) (end 109.22 104.14) (width 0.25) (layer "F.Cu") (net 9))
 (segment (start 121.92 109.22) (end 124.46 109.22) (width 0.25) (layer "F.Cu") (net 9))
 (segment (start 111.76 106.68) (end 119.38 106.68) (width 0.25) (layer "F.Cu") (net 9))
 (segment (start 119.38 106.68) (end 121.92 109.22) (width 0.25) (layer "F.Cu") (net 9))
 (segment (start 109.22 104.14) (end 111.76 106.68) (width 0.25) (layer "F.Cu") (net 9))
 (segment (start 149.86 68.58) (end 162.56 68.58) (width 0.25) (layer "F.Cu") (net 8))
 (segment (start 162.56 88.9) (end 149.86 101.6) (width 0.25) (layer "F.Cu") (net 8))
 (segment (start 149.86 60.96) (end 149.86 68.58) (width 0.25) (layer "F.Cu") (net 8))
 (segment (start 162.56 68.58) (end 162.56 88.9) (width 0.25) (layer "F.Cu") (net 8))
 (segment (start 114.3 91.44) (end 121.92 99.06) (width 0.25) (layer "F.Cu") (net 17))
 (segment (start 109.22 88.9) (end 111.76 91.44) (width 0.25) (layer "F.Cu") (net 17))
 (segment (start 109.22 86.635) (end 109.22 88.9) (width 0.25) (layer "F.Cu") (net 17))
 (segment (start 111.76 91.44) (end 114.3 91.44) (width 0.25) (layer "F.Cu") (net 17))
 (segment (start 121.92 99.06) (end 124.46 99.06) (width 0.25) (layer "F.Cu") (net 17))
 (segment (start 139.7 71.12) (end 160.02 71.12) (width 0.25) (layer "F.Cu") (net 29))
 (segment (start 160.02 71.12) (end 160.02 88.9) (width 0.25) (layer "F.Cu") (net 29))
 (segment (start 160.02 88.9) (end 149.86 99.06) (width 0.25) (layer "F.Cu") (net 29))
 (segment (start 139.7 60.96) (end 139.7 71.12) (width 0.25) (layer "F.Cu") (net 29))
 (segment (start 109.22 99.06) (end 114.3 99.06) (width 0.25) (layer "F.Cu") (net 4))
 (segment (start 109.22 94.255) (end 109.22 99.06) (width 0.25) (layer "F.Cu") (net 4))
 (segment (start 121.92 106.68) (end 124.46 106.68) (width 0.25) (layer "F.Cu") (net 4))
 (segment (start 114.3 99.06) (end 121.92 106.68) (width 0.25) (layer "F.Cu") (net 4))
 (segment (start 109.22 78.74) (end 119.38 88.9) (width 0.25) (layer "F.Cu") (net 16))
 (segment (start 119.38 88.9) (end 119.38 93.98) (width 0.25) (layer "F.Cu") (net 16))
 (segment (start 119.38 93.98) (end 121.92 96.52) (width 0.25) (layer "F.Cu") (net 16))
 (segment (start 121.92 96.52) (end 124.46 96.52) (width 0.25) (layer "F.Cu") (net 16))
 (segment (start 109.22 60.96) (end 109.22 78.74) (width 0.25) (layer "F.Cu") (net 16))
 (segment (start 124.46 114.3) (end 121.92 114.3) (width 0.25) (layer "F.Cu") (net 13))
 (segment (start 116.84 119.38) (end 109.22 119.38) (width 0.25) (layer "F.Cu") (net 13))
 (segment (start 121.92 114.3) (end 116.84 119.38) (width 0.25) (layer "F.Cu") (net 13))
 (segment (start 109.22 119.38) (end 109.22 117.115) (width 0.25) (layer "F.Cu") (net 13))
 (segment (start 157.48 104.14) (end 149.86 111.76) (width 0.25) (layer "F.Cu") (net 11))
 (segment (start 173.16 103.7) (end 172.72 104.14) (width 0.25) (layer "F.Cu") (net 11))
 (segment (start 172.72 104.14) (end 157.48 104.14) (width 0.25) (layer "F.Cu") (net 11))
 (segment (start 173.16 101.875) (end 173.16 103.7) (width 0.25) (layer "F.Cu") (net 11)))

